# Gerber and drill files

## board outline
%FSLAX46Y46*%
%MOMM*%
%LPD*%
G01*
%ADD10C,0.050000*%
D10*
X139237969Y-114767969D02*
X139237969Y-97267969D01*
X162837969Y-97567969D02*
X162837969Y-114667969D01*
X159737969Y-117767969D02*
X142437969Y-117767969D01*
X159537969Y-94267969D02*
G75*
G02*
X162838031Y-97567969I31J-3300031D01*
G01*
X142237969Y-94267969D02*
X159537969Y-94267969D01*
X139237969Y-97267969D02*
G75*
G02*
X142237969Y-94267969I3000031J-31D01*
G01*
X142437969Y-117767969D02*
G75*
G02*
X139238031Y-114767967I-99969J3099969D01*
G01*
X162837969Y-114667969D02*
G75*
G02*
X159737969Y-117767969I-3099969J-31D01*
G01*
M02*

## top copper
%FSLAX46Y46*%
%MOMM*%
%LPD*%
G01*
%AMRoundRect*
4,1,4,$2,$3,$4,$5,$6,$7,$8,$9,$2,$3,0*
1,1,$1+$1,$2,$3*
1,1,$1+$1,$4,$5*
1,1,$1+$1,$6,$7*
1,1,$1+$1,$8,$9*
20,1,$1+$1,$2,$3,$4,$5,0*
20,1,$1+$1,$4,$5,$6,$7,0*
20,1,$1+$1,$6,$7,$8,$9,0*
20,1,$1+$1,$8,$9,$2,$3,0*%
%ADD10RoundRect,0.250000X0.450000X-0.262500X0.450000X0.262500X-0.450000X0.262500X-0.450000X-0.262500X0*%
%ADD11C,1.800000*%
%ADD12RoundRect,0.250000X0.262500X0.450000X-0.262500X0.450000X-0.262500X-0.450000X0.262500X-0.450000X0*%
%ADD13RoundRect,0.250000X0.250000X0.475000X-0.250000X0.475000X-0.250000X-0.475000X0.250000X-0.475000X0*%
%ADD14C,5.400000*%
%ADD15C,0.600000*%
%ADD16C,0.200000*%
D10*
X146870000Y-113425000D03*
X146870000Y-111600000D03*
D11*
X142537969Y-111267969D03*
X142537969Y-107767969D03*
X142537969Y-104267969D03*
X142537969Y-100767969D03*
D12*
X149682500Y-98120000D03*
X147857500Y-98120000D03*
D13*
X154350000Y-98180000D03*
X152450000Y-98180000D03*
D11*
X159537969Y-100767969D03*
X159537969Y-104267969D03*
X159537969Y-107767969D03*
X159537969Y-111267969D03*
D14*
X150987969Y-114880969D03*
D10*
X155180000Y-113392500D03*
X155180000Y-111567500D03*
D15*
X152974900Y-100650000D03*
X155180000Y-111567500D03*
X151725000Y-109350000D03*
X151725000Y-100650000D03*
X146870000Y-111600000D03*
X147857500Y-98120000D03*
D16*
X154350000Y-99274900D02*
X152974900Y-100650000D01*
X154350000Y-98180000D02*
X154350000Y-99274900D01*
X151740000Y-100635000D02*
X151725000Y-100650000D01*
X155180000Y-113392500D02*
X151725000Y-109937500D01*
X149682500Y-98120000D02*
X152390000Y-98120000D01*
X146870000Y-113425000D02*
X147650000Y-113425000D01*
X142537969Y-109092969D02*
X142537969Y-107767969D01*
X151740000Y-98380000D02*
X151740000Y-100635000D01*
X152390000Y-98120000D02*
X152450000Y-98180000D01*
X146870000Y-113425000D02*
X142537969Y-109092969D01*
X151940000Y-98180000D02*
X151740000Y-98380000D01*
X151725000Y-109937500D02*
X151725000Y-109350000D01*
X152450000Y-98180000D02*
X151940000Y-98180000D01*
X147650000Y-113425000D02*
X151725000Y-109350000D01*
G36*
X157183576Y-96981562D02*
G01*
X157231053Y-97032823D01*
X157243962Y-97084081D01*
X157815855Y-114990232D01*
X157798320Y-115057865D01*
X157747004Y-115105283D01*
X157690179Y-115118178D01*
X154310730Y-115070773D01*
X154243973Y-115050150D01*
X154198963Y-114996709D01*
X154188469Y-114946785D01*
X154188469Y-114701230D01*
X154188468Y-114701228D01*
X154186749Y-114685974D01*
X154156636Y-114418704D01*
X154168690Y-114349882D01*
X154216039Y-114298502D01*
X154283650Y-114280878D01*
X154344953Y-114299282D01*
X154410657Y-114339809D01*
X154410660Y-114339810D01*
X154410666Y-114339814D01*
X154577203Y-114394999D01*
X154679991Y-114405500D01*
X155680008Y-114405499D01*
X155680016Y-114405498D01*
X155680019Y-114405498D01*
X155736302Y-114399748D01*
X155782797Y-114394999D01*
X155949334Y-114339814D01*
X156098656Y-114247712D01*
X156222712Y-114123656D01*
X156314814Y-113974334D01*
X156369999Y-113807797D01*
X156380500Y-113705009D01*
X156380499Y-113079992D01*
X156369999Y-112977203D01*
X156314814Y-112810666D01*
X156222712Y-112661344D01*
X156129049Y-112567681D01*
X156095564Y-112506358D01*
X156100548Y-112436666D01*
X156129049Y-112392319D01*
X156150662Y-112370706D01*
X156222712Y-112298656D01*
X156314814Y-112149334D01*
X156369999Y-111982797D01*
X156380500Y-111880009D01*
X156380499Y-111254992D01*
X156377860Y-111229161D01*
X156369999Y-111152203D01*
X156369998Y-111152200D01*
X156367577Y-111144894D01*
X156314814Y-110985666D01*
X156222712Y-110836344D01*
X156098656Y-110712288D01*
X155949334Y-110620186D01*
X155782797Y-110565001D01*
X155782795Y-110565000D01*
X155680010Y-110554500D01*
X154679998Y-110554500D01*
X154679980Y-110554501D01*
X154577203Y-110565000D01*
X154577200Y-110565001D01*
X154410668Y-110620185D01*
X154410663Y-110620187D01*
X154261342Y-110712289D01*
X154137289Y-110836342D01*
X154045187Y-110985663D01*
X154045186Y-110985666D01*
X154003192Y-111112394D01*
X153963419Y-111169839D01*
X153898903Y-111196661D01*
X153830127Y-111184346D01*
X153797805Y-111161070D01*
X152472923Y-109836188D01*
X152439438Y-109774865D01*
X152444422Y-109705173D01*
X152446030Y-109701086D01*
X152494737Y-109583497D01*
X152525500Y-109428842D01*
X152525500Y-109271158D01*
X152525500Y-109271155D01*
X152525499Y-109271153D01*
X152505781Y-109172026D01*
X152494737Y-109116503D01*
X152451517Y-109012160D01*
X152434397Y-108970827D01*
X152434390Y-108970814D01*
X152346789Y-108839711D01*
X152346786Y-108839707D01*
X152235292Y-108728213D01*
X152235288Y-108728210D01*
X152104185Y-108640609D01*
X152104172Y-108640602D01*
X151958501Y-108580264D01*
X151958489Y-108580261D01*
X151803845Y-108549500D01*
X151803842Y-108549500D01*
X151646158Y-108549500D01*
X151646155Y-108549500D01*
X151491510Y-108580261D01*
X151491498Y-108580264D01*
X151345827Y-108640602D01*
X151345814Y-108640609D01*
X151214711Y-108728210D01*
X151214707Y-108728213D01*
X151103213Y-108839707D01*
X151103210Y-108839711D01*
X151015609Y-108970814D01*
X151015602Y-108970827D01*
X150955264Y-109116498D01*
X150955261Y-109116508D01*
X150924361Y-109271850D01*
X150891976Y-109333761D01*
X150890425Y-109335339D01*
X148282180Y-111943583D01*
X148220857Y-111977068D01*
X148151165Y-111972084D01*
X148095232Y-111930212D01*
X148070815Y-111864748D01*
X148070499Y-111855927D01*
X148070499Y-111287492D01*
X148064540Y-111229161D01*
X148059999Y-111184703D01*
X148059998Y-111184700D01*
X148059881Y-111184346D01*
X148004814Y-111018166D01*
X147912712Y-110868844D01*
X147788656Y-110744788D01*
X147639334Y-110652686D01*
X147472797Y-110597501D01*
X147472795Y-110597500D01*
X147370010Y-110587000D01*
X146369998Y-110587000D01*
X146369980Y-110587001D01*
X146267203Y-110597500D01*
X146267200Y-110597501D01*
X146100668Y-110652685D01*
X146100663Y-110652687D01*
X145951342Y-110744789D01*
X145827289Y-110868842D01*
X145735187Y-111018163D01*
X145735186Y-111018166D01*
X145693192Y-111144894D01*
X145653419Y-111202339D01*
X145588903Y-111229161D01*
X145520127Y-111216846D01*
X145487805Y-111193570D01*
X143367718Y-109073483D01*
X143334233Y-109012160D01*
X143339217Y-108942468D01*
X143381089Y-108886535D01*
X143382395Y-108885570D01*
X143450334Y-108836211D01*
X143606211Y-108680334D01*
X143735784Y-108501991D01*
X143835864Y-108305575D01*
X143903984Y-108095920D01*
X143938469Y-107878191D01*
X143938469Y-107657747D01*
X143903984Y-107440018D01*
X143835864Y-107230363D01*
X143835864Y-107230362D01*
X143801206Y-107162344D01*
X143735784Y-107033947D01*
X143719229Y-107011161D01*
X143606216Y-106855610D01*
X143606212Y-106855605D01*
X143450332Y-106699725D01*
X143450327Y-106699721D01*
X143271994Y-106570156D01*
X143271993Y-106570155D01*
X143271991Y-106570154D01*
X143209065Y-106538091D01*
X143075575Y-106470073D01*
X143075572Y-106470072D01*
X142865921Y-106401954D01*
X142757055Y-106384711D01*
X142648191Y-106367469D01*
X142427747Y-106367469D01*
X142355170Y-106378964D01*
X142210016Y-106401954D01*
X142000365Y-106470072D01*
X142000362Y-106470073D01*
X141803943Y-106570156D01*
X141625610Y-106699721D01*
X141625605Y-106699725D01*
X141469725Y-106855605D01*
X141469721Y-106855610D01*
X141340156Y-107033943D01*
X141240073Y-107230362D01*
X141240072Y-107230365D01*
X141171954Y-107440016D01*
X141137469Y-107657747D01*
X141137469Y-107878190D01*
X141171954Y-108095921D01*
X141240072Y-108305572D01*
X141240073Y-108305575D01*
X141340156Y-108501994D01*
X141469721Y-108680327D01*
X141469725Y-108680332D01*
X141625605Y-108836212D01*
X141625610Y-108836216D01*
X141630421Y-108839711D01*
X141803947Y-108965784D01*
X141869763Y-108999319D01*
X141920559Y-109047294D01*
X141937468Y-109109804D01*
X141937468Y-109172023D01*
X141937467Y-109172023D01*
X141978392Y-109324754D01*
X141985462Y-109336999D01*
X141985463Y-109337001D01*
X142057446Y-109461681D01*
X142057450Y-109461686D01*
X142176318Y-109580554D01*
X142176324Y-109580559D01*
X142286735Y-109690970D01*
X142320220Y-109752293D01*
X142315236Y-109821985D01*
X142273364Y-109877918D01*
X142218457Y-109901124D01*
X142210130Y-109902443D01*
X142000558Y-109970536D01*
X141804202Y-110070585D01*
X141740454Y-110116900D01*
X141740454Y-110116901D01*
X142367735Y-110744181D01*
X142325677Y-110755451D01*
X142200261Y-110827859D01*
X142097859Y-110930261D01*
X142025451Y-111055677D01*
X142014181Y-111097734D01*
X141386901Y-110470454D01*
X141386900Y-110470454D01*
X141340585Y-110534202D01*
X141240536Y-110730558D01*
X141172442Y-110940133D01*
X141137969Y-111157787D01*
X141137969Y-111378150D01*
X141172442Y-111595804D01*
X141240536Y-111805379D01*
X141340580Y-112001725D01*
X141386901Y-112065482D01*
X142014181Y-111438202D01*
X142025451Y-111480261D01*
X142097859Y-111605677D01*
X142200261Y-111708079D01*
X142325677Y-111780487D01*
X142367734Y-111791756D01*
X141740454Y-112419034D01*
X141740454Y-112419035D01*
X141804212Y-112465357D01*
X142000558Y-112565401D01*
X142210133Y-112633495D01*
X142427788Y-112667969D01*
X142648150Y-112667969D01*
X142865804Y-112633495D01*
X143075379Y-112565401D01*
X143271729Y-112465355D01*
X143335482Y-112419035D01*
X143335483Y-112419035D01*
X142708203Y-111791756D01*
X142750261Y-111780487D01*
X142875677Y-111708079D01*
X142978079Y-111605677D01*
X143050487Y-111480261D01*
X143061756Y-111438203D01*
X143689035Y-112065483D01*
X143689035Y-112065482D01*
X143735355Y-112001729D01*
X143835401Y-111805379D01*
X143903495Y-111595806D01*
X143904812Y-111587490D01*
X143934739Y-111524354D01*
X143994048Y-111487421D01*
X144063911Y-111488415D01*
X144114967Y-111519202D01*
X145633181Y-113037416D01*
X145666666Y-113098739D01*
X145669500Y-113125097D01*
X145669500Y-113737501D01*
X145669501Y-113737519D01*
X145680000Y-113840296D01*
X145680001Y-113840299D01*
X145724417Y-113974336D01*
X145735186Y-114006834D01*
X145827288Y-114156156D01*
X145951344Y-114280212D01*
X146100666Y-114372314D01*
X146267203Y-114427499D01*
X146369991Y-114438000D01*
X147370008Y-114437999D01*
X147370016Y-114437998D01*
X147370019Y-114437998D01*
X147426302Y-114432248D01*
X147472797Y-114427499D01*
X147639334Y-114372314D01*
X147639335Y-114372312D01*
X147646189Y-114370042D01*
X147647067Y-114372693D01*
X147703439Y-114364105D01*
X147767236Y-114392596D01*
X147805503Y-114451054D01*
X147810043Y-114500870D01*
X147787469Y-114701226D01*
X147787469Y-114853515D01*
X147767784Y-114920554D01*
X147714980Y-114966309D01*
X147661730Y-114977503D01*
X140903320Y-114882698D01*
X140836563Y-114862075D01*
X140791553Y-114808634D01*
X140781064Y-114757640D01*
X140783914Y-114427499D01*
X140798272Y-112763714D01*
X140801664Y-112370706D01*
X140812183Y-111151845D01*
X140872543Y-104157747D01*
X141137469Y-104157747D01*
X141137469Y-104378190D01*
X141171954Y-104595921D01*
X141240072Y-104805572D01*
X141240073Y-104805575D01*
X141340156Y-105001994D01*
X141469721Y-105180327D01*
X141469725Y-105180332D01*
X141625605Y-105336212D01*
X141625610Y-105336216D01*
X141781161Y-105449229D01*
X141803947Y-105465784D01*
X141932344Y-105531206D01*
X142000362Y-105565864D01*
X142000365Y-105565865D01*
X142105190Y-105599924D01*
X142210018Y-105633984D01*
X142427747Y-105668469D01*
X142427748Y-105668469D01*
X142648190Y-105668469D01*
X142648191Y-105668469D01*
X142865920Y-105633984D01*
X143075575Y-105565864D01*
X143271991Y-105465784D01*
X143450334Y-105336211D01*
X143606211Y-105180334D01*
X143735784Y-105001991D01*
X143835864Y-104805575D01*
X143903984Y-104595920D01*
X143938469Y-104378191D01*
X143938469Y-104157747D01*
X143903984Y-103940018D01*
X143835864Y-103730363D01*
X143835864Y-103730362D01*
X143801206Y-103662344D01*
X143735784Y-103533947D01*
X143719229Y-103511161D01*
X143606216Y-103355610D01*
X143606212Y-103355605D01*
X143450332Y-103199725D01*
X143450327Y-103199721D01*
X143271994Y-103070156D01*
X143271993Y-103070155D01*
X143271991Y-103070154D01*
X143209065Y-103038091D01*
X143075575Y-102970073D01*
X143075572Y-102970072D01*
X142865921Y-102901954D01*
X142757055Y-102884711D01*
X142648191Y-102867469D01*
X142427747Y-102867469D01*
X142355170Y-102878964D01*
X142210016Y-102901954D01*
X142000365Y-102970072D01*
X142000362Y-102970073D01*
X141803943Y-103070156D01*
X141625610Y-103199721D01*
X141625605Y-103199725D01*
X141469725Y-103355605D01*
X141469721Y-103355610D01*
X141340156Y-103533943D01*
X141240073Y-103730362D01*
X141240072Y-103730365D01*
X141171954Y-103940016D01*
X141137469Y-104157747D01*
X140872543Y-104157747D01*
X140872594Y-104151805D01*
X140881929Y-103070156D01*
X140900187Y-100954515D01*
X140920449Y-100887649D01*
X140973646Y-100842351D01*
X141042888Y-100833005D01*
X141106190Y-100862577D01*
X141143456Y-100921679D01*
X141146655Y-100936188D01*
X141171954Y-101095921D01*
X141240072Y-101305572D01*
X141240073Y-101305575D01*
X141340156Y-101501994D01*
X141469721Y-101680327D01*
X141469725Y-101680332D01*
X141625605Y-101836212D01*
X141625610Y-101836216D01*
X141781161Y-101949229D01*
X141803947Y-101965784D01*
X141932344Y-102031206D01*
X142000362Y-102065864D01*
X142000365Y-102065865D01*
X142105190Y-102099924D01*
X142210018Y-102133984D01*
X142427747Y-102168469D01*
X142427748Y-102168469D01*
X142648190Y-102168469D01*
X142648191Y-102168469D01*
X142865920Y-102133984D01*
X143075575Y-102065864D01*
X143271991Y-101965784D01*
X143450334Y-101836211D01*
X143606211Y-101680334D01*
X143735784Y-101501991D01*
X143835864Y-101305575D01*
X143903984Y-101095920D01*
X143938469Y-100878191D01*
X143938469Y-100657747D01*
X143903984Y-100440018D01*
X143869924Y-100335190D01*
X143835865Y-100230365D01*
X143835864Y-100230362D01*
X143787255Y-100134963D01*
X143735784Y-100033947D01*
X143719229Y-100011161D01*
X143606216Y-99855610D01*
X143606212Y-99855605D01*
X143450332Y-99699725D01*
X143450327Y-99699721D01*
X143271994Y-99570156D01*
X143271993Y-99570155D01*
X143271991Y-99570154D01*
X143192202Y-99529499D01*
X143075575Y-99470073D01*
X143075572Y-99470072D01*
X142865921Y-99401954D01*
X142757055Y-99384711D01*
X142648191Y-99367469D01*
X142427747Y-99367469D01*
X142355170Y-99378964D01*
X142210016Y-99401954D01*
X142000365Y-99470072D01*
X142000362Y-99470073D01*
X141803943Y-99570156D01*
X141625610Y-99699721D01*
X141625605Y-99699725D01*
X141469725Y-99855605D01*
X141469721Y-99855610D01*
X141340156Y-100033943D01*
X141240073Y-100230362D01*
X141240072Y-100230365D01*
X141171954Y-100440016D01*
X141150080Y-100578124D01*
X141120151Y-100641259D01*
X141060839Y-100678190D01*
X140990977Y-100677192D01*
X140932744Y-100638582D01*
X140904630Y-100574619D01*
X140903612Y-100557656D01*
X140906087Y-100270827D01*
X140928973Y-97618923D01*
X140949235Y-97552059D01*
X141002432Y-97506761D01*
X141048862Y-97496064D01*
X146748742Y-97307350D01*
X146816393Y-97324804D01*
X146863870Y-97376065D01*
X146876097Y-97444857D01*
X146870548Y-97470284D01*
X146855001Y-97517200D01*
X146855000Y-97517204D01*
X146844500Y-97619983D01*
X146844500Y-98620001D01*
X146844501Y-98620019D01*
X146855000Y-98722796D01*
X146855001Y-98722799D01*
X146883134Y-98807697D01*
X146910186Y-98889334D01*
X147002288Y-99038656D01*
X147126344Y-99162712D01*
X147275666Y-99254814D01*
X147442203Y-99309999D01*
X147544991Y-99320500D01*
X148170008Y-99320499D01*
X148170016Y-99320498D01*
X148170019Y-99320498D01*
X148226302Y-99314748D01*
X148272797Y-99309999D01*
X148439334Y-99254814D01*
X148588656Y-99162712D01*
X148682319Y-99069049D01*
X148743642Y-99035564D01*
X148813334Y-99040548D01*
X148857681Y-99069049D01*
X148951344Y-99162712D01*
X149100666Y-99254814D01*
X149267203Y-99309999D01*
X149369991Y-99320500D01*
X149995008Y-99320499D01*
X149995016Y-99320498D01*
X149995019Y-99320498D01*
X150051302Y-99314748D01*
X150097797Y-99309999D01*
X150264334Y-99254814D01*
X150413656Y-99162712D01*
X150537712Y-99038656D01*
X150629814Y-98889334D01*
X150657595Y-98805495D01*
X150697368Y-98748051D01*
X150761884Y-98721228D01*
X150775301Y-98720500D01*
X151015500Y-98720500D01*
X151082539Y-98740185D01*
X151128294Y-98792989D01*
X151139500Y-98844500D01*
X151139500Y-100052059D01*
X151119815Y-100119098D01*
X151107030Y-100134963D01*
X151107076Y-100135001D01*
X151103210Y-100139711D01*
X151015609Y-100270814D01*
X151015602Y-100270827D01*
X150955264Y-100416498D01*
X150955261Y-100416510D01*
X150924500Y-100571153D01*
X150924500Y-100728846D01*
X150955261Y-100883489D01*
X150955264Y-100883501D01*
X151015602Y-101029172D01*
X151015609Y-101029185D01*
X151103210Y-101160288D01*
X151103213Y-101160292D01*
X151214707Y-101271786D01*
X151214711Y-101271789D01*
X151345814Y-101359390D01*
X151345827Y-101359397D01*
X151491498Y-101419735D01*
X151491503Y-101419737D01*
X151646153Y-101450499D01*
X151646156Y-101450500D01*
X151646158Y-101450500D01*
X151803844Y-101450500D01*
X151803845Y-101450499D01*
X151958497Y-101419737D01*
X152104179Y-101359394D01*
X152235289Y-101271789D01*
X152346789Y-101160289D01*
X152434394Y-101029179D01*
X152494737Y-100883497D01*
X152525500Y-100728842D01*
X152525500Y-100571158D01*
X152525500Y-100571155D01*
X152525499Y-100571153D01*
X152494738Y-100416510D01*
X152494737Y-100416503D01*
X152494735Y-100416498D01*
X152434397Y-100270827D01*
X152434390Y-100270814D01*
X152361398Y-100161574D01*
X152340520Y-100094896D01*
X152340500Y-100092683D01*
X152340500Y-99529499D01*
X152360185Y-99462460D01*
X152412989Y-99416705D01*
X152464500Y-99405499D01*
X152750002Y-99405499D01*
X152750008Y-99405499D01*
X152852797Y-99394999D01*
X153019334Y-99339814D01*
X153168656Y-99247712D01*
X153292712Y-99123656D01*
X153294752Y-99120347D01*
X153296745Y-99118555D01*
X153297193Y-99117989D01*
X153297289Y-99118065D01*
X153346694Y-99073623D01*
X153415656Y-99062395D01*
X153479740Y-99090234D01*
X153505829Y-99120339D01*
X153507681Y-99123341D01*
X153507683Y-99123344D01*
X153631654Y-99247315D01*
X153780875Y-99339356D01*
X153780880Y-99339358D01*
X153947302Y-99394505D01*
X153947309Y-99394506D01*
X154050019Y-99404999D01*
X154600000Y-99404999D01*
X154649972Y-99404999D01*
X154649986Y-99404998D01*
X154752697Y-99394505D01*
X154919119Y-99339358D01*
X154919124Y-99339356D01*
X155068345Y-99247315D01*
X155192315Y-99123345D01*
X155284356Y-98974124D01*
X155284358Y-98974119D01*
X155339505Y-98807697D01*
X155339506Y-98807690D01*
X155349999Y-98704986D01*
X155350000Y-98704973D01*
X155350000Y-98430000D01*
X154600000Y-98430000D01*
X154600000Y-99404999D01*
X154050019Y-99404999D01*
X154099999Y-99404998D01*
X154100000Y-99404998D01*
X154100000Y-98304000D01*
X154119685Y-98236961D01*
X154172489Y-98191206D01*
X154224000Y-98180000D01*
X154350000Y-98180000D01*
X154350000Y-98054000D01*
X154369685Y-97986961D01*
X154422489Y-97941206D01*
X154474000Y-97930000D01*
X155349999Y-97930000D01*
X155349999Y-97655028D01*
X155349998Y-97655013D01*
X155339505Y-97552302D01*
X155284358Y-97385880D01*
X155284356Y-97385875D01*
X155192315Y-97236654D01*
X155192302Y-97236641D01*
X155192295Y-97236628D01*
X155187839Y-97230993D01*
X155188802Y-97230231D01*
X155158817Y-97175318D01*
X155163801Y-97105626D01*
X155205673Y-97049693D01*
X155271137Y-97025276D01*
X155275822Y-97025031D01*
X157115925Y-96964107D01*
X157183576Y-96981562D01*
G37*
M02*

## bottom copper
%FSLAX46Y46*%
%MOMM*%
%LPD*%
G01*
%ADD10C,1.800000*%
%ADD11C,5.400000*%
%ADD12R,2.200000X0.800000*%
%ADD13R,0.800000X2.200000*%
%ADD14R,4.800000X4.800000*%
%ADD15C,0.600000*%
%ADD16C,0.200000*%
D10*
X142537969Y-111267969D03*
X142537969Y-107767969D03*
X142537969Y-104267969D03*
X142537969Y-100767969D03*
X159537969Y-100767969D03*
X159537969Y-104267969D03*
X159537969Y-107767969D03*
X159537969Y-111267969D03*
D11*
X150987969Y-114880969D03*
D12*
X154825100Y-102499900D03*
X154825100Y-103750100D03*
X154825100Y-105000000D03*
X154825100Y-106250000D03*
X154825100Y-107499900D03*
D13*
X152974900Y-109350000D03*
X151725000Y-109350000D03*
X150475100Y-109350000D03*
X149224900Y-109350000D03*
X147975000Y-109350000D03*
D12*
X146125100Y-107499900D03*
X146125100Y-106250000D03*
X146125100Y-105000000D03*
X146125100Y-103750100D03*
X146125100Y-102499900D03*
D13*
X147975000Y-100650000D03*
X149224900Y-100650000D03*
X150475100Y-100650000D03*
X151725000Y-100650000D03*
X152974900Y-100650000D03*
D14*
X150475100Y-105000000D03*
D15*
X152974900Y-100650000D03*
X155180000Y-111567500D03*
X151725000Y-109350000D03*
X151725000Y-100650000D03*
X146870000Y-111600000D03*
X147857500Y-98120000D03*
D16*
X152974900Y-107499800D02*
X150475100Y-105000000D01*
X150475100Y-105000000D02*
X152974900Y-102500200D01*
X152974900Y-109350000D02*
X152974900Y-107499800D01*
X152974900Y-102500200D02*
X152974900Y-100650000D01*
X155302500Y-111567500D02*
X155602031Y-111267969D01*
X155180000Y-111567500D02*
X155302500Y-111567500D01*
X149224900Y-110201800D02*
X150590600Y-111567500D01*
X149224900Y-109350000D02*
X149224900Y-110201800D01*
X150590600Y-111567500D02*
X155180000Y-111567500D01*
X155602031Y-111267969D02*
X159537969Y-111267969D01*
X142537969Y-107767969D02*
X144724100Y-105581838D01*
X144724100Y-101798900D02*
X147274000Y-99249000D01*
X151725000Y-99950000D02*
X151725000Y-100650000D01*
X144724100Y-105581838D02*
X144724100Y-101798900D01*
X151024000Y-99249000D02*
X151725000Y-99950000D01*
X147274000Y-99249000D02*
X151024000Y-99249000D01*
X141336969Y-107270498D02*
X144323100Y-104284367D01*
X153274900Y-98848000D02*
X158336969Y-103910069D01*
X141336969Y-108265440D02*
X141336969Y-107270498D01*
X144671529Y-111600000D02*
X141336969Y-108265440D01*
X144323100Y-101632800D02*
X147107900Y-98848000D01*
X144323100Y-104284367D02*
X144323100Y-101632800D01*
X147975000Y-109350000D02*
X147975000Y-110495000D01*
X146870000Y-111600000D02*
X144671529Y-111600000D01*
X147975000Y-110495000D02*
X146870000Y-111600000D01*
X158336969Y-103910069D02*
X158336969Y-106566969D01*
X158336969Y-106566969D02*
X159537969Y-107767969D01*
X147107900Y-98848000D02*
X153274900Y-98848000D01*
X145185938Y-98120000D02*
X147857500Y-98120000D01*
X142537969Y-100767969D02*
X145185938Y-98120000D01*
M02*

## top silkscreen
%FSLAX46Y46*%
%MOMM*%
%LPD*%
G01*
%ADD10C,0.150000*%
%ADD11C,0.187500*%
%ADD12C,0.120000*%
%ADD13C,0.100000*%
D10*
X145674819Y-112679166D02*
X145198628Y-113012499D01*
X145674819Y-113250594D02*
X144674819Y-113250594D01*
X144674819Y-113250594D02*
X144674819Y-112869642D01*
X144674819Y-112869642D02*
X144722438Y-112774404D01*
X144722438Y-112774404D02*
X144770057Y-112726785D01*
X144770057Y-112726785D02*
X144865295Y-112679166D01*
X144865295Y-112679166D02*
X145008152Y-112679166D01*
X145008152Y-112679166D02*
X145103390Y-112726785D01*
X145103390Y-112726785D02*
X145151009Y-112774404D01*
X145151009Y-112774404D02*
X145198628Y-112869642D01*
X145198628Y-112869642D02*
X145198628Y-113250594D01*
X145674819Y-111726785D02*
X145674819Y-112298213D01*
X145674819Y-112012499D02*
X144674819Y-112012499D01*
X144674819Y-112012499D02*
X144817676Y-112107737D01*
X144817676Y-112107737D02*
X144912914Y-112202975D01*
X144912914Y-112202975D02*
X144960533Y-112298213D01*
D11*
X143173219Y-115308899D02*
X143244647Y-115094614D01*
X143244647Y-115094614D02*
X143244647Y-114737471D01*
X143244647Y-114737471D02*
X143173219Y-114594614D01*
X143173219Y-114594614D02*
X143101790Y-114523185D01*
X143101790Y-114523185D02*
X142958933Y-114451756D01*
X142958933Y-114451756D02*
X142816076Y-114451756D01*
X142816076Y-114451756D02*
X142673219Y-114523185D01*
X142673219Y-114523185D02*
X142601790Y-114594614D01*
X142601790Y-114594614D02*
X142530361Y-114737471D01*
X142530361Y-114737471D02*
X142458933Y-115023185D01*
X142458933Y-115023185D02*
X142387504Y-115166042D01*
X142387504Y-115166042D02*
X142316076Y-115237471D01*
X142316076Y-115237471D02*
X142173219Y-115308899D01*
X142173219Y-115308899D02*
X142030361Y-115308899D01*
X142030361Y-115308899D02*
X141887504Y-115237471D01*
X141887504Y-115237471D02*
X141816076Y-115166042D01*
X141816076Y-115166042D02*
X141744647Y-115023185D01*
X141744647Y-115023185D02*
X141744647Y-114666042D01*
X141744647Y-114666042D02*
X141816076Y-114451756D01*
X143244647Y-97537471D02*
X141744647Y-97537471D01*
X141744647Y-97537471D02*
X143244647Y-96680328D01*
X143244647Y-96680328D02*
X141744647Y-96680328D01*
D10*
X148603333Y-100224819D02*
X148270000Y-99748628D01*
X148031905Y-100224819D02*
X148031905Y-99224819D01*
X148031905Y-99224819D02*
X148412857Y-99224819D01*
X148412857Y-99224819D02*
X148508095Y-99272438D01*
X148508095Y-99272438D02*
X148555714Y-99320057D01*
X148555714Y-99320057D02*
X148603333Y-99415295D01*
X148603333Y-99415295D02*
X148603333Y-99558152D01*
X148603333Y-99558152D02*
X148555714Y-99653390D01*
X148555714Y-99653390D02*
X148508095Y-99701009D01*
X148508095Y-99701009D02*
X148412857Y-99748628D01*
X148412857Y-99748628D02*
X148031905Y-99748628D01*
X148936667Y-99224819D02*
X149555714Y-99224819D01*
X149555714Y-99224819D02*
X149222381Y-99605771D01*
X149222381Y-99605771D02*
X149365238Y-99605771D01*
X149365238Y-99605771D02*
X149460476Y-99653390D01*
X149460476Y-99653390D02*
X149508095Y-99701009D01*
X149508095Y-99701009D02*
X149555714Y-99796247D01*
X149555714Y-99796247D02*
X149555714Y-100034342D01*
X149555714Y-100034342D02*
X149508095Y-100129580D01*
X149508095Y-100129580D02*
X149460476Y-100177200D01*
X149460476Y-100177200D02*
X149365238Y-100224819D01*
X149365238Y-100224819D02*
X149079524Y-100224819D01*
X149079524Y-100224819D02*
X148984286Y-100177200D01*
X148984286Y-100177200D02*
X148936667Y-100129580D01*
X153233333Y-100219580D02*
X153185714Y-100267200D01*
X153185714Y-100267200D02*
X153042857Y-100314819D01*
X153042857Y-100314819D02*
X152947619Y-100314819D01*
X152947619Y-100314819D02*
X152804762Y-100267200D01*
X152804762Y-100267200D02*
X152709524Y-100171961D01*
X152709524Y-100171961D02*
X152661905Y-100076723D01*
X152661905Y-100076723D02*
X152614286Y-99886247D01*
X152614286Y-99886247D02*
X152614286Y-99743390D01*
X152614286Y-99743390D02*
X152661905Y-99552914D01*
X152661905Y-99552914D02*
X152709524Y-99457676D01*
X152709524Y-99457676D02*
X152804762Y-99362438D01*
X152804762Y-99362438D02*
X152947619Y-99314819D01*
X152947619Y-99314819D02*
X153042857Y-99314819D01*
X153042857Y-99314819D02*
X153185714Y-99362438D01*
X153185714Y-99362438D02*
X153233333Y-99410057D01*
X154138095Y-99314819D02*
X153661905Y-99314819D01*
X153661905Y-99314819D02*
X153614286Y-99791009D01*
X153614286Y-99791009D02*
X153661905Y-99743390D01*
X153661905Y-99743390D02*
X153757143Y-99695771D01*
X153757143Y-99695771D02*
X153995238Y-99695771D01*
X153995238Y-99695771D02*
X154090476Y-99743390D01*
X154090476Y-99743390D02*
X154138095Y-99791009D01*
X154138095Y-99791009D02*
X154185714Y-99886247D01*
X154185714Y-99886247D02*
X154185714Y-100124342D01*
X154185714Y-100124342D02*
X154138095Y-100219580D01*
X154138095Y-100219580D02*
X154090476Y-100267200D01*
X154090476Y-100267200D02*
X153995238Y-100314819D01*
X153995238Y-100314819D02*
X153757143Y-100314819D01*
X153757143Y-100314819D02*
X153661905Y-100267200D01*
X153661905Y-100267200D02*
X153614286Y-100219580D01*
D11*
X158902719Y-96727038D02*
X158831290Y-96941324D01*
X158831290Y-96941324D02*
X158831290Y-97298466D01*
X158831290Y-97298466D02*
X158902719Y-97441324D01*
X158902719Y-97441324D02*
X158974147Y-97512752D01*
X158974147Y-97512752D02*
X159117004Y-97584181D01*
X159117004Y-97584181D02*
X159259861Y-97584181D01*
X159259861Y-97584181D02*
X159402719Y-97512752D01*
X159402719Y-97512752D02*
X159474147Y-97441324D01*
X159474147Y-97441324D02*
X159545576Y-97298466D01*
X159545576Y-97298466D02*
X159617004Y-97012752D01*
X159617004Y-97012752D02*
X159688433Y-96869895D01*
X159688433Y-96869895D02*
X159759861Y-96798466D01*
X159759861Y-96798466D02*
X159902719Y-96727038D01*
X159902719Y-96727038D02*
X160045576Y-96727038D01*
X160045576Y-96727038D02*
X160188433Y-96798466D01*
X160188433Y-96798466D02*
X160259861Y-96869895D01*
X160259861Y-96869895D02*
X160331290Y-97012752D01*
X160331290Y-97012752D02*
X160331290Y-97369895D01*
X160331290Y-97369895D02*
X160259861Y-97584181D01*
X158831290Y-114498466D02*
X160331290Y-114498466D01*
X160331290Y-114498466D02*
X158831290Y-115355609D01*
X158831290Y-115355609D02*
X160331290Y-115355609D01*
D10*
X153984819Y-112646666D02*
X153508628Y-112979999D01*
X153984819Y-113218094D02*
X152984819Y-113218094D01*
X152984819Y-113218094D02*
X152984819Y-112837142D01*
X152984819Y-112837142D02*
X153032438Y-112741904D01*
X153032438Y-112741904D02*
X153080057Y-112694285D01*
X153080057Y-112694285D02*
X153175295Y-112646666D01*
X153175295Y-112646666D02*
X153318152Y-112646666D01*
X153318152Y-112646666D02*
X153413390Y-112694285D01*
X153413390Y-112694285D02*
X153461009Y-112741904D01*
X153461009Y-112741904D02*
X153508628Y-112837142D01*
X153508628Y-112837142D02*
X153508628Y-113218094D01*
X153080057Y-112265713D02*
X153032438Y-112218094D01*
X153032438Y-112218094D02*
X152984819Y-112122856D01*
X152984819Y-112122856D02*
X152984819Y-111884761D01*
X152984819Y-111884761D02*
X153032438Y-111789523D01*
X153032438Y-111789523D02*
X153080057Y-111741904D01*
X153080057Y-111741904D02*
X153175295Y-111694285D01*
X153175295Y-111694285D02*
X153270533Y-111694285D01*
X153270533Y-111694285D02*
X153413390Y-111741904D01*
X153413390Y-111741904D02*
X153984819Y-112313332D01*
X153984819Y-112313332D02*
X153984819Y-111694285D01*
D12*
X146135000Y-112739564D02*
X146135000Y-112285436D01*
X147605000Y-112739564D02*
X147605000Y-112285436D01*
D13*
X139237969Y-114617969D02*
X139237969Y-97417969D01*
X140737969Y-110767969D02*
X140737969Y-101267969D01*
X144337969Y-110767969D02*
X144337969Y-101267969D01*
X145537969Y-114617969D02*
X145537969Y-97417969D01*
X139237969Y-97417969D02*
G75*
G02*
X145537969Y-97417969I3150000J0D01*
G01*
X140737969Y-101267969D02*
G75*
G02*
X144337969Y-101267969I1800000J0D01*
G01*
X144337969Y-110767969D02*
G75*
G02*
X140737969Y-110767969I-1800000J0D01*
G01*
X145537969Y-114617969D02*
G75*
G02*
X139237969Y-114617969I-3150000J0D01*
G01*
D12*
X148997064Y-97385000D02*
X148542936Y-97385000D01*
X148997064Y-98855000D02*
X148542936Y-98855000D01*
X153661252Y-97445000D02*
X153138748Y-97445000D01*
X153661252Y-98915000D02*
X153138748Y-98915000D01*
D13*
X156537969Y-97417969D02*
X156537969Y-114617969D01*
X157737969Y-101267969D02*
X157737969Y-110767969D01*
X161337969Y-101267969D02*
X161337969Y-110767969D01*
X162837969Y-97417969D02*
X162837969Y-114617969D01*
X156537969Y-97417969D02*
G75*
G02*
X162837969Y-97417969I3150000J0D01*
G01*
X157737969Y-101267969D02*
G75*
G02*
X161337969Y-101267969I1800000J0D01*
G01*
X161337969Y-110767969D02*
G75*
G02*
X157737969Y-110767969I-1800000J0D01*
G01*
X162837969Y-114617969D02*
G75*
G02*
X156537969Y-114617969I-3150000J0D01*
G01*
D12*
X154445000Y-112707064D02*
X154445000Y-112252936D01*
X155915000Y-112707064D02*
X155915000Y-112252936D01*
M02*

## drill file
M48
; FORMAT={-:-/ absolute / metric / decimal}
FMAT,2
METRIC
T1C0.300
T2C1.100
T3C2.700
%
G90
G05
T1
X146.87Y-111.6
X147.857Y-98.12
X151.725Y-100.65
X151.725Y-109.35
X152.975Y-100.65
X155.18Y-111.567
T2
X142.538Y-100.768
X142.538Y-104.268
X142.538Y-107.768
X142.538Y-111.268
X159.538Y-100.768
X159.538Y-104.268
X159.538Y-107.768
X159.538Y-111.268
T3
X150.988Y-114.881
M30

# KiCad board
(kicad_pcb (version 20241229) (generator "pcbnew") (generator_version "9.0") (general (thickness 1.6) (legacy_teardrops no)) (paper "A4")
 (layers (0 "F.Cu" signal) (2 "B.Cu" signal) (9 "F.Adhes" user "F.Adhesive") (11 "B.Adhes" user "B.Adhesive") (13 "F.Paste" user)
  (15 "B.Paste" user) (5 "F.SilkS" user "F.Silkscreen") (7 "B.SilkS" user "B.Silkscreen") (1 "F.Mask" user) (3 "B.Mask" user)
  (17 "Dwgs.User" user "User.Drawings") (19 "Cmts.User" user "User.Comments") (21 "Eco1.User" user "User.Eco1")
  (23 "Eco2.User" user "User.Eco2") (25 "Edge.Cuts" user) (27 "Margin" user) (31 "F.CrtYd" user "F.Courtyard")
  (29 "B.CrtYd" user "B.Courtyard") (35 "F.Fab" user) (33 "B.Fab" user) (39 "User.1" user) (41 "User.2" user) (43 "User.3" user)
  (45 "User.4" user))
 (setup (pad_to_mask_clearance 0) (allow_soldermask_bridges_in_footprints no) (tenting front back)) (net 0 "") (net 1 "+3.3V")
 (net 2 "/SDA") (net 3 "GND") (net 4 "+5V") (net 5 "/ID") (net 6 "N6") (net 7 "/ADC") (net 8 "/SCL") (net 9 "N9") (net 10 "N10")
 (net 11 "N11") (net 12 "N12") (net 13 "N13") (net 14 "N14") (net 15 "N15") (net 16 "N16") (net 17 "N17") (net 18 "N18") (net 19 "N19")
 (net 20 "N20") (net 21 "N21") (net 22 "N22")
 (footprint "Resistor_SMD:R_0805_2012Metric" (layer "F.Cu") (at 146.87 112.5125 90)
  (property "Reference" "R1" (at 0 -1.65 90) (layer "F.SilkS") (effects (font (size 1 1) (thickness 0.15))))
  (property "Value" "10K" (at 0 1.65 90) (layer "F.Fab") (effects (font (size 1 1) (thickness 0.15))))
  (fp_line (start -0.227064 -0.735) (end 0.227064 -0.735) (stroke (width 0.12) (type solid)) (layer "F.SilkS"))
  (fp_line (start -0.227064 0.735) (end 0.227064 0.735) (stroke (width 0.12) (type solid)) (layer "F.SilkS"))
  (pad "1" smd roundrect (at -0.9125 0 90) (size 1.025 1.4) (layers "F.Cu" "F.Mask" "F.Paste") (roundrect_rratio 0.243902) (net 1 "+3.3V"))
  (pad "2" smd roundrect (at 0.9125 0 90) (size 1.025 1.4) (layers "F.Cu" "F.Mask" "F.Paste") (roundrect_rratio 0.243902) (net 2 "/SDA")))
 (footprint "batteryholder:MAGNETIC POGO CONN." (layer "F.Cu") (at 142.537969 106.017969 90)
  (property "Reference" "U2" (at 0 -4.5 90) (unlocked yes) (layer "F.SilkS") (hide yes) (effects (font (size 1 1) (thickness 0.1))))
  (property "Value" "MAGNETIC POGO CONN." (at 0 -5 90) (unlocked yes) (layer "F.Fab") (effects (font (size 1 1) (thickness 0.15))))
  (fp_line (start -8.6 -3.3) (end 8.6 -3.3) (stroke (width 0.1) (type default)) (layer "F.SilkS"))
  (fp_line (start -4.75 -1.8) (end 4.75 -1.8) (stroke (width 0.1) (type default)) (layer "F.SilkS"))
  (fp_line (start -4.75 1.8) (end 4.75 1.8) (stroke (width 0.1) (type default)) (layer "F.SilkS"))
  (fp_line (start -8.6 3) (end 8.6 3) (stroke (width 0.1) (type default)) (layer "F.SilkS"))
  (fp_arc (start 8.6 -3.3) (mid 11.75 -0.15) (end 8.6 3) (stroke (width 0.1) (type default)) (layer "F.SilkS"))
  (fp_arc (start 4.75 -1.8) (mid 6.55 0) (end 4.75 1.8) (stroke (width 0.1) (type default)) (layer "F.SilkS"))
  (fp_arc (start -4.75 1.8) (mid -6.55 0) (end -4.75 -1.8) (stroke (width 0.1) (type default)) (layer "F.SilkS"))
  (fp_arc (start -8.6 3) (mid -11.75 -0.15) (end -8.6 -3.3) (stroke (width 0.1) (type default)) (layer "F.SilkS"))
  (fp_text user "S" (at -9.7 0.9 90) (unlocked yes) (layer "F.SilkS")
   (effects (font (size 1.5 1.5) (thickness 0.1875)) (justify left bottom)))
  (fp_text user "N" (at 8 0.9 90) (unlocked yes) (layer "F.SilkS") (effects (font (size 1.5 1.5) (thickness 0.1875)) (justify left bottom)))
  (pad "1" thru_hole circle (at -5.25 0 90) (size 1.8 1.8) (drill 1.1) (layers "*.Cu" "*.Mask") (remove_unused_layers no) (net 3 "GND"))
  (pad "2" thru_hole circle (at -1.75 0 90) (size 1.8 1.8) (drill 1.1) (layers "*.Cu" "*.Mask") (remove_unused_layers no) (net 1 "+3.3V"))
  (pad "3" thru_hole circle (at 1.75 0 90) (size 1.8 1.8) (drill 1.1) (layers "*.Cu" "*.Mask") (remove_unused_layers no) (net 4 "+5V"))
  (pad "4" thru_hole circle (at 5.25 0 90) (size 1.8 1.8) (drill 1.1) (layers "*.Cu" "*.Mask") (remove_unused_layers no) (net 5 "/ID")))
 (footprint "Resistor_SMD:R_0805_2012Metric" (layer "F.Cu") (at 148.77 98.12 180)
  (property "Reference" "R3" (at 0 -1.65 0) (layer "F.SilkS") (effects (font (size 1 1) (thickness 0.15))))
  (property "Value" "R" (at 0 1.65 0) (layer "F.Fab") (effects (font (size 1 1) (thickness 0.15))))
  (fp_line (start -0.227064 0.735) (end 0.227064 0.735) (stroke (width 0.12) (type solid)) (layer "F.SilkS"))
  (fp_line (start -0.227064 -0.735) (end 0.227064 -0.735) (stroke (width 0.12) (type solid)) (layer "F.SilkS"))
  (pad "1" smd roundrect (at -0.9125 0 180) (size 1.025 1.4) (layers "F.Cu" "F.Mask" "F.Paste") (roundrect_rratio 0.243902) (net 1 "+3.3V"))
  (pad "2" smd roundrect (at 0.9125 0 180) (size 1.025 1.4) (layers "F.Cu" "F.Mask" "F.Paste") (roundrect_rratio 0.243902) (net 5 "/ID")))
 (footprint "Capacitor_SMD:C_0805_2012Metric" (layer "F.Cu") (at 153.4 98.18 180)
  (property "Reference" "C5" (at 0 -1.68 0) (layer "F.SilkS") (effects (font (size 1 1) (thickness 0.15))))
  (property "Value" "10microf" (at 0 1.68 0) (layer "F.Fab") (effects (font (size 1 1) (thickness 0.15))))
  (fp_line (start -0.261252 0.735) (end 0.261252 0.735) (stroke (width 0.12) (type solid)) (layer "F.SilkS"))
  (fp_line (start -0.261252 -0.735) (end 0.261252 -0.735) (stroke (width 0.12) (type solid)) (layer "F.SilkS"))
  (pad "1" smd roundrect (at -0.95 0 180) (size 1 1.45) (layers "F.Cu" "F.Mask" "F.Paste") (roundrect_rratio 0.25) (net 3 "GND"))
  (pad "2" smd roundrect (at 0.95 0 180) (size 1 1.45) (layers "F.Cu" "F.Mask" "F.Paste") (roundrect_rratio 0.25) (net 1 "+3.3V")))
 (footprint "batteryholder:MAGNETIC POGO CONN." (layer "F.Cu") (at 159.537969 106.017969 -90)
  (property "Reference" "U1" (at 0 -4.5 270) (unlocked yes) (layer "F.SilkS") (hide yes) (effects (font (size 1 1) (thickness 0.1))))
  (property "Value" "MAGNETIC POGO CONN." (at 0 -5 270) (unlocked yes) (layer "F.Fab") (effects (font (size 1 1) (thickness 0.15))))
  (fp_line (start -8.6 3) (end 8.6 3) (stroke (width 0.1) (type default)) (layer "F.SilkS"))
  (fp_line (start -4.75 1.8) (end 4.75 1.8) (stroke (width 0.1) (type default)) (layer "F.SilkS"))
  (fp_line (start -4.75 -1.8) (end 4.75 -1.8) (stroke (width 0.1) (type default)) (layer "F.SilkS"))
  (fp_line (start -8.6 -3.3) (end 8.6 -3.3) (stroke (width 0.1) (type default)) (layer "F.SilkS"))
  (fp_arc (start -8.6 3) (mid -11.75 -0.15) (end -8.6 -3.3) (stroke (width 0.1) (type default)) (layer "F.SilkS"))
  (fp_arc (start -4.75 1.8) (mid -6.55 0) (end -4.75 -1.8) (stroke (width 0.1) (type default)) (layer "F.SilkS"))
  (fp_arc (start 4.75 -1.8) (mid 6.55 0) (end 4.75 1.8) (stroke (width 0.1) (type default)) (layer "F.SilkS"))
  (fp_arc (start 8.6 -3.3) (mid 11.75 -0.15) (end 8.6 3) (stroke (width 0.1) (type default)) (layer "F.SilkS"))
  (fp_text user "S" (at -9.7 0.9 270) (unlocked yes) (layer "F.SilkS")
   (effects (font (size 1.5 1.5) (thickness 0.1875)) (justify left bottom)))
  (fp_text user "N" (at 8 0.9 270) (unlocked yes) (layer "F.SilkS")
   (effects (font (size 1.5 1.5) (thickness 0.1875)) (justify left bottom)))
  (pad "1" thru_hole circle (at -5.25 0 270) (size 1.8 1.8) (drill 1.1) (layers "*.Cu" "*.Mask") (remove_unused_layers no) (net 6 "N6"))
  (pad "2" thru_hole circle (at -1.75 0 270) (size 1.8 1.8) (drill 1.1) (layers "*.Cu" "*.Mask") (remove_unused_layers no) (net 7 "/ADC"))
  (pad "3" thru_hole circle (at 1.75 0 270) (size 1.8 1.8) (drill 1.1) (layers "*.Cu" "*.Mask") (remove_unused_layers no) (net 2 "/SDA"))
  (pad "4" thru_hole circle (at 5.25 0 270) (size 1.8 1.8) (drill 1.1) (layers "*.Cu" "*.Mask") (remove_unused_layers no) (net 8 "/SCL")))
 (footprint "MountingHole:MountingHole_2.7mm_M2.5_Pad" (layer "F.Cu") (at 150.987969 114.880969)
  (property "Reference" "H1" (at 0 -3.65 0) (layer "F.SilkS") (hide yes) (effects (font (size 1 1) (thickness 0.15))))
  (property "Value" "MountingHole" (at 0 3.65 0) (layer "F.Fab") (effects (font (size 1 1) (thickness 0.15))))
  (pad "1" thru_hole circle (at 0 0) (size 5.4 5.4) (drill 2.7) (layers "*.Cu" "*.Mask") (remove_unused_layers no) (zone_connect 2)))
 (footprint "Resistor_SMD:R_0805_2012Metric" (layer "F.Cu") (at 155.18 112.48 90)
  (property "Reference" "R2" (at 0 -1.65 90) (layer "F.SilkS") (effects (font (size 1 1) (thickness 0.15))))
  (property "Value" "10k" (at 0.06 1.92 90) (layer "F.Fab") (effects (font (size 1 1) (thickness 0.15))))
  (fp_line (start -0.227064 -0.735) (end 0.227064 -0.735) (stroke (width 0.12) (type solid)) (layer "F.SilkS"))
  (fp_line (start -0.227064 0.735) (end 0.227064 0.735) (stroke (width 0.12) (type solid)) (layer "F.SilkS"))
  (pad "1" smd roundrect (at -0.9125 0 90) (size 1.025 1.4) (layers "F.Cu" "F.Mask" "F.Paste") (roundrect_rratio 0.243902) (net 1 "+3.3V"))
  (pad "2" smd roundrect (at 0.9125 0 90) (size 1.025 1.4) (layers "F.Cu" "F.Mask" "F.Paste") (roundrect_rratio 0.243902) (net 8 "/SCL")))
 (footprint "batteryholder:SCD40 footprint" (layer "B.Cu") (at 150.475 105 180)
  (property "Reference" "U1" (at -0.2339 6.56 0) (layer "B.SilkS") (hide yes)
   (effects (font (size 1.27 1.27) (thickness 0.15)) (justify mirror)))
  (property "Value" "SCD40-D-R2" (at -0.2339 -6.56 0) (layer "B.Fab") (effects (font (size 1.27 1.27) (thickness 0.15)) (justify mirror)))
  (pad "1" smd rect (at -4.3501 2.5001 180) (size 2.2 0.8) (layers "B.Cu" "B.Mask" "B.Paste") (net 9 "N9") (solder_mask_margin 0.05)
   (solder_paste_margin 0) (thermal_bridge_angle 0))
  (pad "2" smd rect (at -4.3501 1.2499 180) (size 2.2 0.8) (layers "B.Cu" "B.Mask" "B.Paste") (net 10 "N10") (solder_mask_margin 0.05)
   (solder_paste_margin 0) (thermal_bridge_angle 0))
  (pad "3" smd rect (at -4.3501 0 180) (size 2.2 0.8) (layers "B.Cu" "B.Mask" "B.Paste") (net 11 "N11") (solder_mask_margin 0.05)
   (solder_paste_margin 0) (thermal_bridge_angle 0))
  (pad "4" smd rect (at -4.3501 -1.25 180) (size 2.2 0.8) (layers "B.Cu" "B.Mask" "B.Paste") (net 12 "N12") (solder_mask_margin 0.05)
   (solder_paste_margin 0) (thermal_bridge_angle 0))
  (pad "5" smd rect (at -4.3501 -2.4999 180) (size 2.2 0.8) (layers "B.Cu" "B.Mask" "B.Paste") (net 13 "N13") (solder_mask_margin 0.05)
   (solder_paste_margin 0) (thermal_bridge_angle 0))
  (pad "6" smd rect (at -2.4999 -4.35 90) (size 2.2 0.8) (layers "B.Cu" "B.Mask" "B.Paste") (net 3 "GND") (solder_mask_margin 0.05)
   (solder_paste_margin 0) (thermal_bridge_angle 0))
  (pad "7" smd rect (at -1.25 -4.35 90) (size 2.2 0.8) (layers "B.Cu" "B.Mask" "B.Paste") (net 1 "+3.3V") (solder_mask_margin 0.05)
   (solder_paste_margin 0) (thermal_bridge_angle 0))
  (pad "8" smd rect (at -0.0001 -4.35 90) (size 2.2 0.8) (layers "B.Cu" "B.Mask" "B.Paste") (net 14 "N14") (solder_mask_margin 0.05)
   (solder_paste_margin 0) (thermal_bridge_angle 0))
  (pad "9" smd rect (at 1.2501 -4.35 90) (size 2.2 0.8) (layers "B.Cu" "B.Mask" "B.Paste") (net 8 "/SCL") (solder_mask_margin 0.05)
   (solder_paste_margin 0) (thermal_bridge_angle 0))
  (pad "10" smd rect (at 2.5 -4.35 90) (size 2.2 0.8) (layers "B.Cu" "B.Mask" "B.Paste") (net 2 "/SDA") (solder_mask_margin 0.05)
   (solder_paste_margin 0) (thermal_bridge_angle 0))
  (pad "11" smd rect (at 4.3499 -2.4999) (size 2.2 0.8) (layers "B.Cu" "B.Mask" "B.Paste") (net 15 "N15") (solder_mask_margin 0.05)
   (solder_paste_margin 0) (thermal_bridge_angle 0))
  (pad "12" smd rect (at 4.3499 -1.25) (size 2.2 0.8) (layers "B.Cu" "B.Mask" "B.Paste") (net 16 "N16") (solder_mask_margin 0.05)
   (solder_paste_margin 0) (thermal_bridge_angle 0))
  (pad "13" smd rect (at 4.3499 0) (size 2.2 0.8) (layers "B.Cu" "B.Mask" "B.Paste") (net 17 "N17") (solder_mask_margin 0.05)
   (solder_paste_margin 0) (thermal_bridge_angle 0))
  (pad "14" smd rect (at 4.3499 1.2499) (size 2.2 0.8) (layers "B.Cu" "B.Mask" "B.Paste") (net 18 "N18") (solder_mask_margin 0.05)
   (solder_paste_margin 0) (thermal_bridge_angle 0))
  (pad "15" smd rect (at 4.3499 2.5001) (size 2.2 0.8) (layers "B.Cu" "B.Mask" "B.Paste") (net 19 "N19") (solder_mask_margin 0.05)
   (solder_paste_margin 0) (thermal_bridge_angle 0))
  (pad "16" smd rect (at 2.5 4.35 270) (size 2.2 0.8) (layers "B.Cu" "B.Mask" "B.Paste") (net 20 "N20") (solder_mask_margin 0.05)
   (solder_paste_margin 0) (thermal_bridge_angle 0))
  (pad "17" smd rect (at 1.2501 4.35 270) (size 2.2 0.8) (layers "B.Cu" "B.Mask" "B.Paste") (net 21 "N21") (solder_mask_margin 0.05)
   (solder_paste_margin 0) (thermal_bridge_angle 0))
  (pad "18" smd rect (at -0.0001 4.35 270) (size 2.2 0.8) (layers "B.Cu" "B.Mask" "B.Paste") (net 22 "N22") (solder_mask_margin 0.05)
   (solder_paste_margin 0) (thermal_bridge_angle 0))
  (pad "19" smd rect (at -1.25 4.35 270) (size 2.2 0.8) (layers "B.Cu" "B.Mask" "B.Paste") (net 1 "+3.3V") (solder_mask_margin 0.05)
   (solder_paste_margin 0) (thermal_bridge_angle 0))
  (pad "20" smd rect (at -2.4999 4.35 270) (size 2.2 0.8) (layers "B.Cu" "B.Mask" "B.Paste") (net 3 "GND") (solder_mask_margin 0.05)
   (solder_paste_margin 0) (thermal_bridge_angle 0))
  (pad "21" smd rect (at -0.0001 0 90) (size 4.8 4.8) (layers "B.Cu" "B.Mask" "B.Paste") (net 3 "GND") (solder_mask_margin 0.05)
   (solder_paste_margin 0) (thermal_bridge_angle 0))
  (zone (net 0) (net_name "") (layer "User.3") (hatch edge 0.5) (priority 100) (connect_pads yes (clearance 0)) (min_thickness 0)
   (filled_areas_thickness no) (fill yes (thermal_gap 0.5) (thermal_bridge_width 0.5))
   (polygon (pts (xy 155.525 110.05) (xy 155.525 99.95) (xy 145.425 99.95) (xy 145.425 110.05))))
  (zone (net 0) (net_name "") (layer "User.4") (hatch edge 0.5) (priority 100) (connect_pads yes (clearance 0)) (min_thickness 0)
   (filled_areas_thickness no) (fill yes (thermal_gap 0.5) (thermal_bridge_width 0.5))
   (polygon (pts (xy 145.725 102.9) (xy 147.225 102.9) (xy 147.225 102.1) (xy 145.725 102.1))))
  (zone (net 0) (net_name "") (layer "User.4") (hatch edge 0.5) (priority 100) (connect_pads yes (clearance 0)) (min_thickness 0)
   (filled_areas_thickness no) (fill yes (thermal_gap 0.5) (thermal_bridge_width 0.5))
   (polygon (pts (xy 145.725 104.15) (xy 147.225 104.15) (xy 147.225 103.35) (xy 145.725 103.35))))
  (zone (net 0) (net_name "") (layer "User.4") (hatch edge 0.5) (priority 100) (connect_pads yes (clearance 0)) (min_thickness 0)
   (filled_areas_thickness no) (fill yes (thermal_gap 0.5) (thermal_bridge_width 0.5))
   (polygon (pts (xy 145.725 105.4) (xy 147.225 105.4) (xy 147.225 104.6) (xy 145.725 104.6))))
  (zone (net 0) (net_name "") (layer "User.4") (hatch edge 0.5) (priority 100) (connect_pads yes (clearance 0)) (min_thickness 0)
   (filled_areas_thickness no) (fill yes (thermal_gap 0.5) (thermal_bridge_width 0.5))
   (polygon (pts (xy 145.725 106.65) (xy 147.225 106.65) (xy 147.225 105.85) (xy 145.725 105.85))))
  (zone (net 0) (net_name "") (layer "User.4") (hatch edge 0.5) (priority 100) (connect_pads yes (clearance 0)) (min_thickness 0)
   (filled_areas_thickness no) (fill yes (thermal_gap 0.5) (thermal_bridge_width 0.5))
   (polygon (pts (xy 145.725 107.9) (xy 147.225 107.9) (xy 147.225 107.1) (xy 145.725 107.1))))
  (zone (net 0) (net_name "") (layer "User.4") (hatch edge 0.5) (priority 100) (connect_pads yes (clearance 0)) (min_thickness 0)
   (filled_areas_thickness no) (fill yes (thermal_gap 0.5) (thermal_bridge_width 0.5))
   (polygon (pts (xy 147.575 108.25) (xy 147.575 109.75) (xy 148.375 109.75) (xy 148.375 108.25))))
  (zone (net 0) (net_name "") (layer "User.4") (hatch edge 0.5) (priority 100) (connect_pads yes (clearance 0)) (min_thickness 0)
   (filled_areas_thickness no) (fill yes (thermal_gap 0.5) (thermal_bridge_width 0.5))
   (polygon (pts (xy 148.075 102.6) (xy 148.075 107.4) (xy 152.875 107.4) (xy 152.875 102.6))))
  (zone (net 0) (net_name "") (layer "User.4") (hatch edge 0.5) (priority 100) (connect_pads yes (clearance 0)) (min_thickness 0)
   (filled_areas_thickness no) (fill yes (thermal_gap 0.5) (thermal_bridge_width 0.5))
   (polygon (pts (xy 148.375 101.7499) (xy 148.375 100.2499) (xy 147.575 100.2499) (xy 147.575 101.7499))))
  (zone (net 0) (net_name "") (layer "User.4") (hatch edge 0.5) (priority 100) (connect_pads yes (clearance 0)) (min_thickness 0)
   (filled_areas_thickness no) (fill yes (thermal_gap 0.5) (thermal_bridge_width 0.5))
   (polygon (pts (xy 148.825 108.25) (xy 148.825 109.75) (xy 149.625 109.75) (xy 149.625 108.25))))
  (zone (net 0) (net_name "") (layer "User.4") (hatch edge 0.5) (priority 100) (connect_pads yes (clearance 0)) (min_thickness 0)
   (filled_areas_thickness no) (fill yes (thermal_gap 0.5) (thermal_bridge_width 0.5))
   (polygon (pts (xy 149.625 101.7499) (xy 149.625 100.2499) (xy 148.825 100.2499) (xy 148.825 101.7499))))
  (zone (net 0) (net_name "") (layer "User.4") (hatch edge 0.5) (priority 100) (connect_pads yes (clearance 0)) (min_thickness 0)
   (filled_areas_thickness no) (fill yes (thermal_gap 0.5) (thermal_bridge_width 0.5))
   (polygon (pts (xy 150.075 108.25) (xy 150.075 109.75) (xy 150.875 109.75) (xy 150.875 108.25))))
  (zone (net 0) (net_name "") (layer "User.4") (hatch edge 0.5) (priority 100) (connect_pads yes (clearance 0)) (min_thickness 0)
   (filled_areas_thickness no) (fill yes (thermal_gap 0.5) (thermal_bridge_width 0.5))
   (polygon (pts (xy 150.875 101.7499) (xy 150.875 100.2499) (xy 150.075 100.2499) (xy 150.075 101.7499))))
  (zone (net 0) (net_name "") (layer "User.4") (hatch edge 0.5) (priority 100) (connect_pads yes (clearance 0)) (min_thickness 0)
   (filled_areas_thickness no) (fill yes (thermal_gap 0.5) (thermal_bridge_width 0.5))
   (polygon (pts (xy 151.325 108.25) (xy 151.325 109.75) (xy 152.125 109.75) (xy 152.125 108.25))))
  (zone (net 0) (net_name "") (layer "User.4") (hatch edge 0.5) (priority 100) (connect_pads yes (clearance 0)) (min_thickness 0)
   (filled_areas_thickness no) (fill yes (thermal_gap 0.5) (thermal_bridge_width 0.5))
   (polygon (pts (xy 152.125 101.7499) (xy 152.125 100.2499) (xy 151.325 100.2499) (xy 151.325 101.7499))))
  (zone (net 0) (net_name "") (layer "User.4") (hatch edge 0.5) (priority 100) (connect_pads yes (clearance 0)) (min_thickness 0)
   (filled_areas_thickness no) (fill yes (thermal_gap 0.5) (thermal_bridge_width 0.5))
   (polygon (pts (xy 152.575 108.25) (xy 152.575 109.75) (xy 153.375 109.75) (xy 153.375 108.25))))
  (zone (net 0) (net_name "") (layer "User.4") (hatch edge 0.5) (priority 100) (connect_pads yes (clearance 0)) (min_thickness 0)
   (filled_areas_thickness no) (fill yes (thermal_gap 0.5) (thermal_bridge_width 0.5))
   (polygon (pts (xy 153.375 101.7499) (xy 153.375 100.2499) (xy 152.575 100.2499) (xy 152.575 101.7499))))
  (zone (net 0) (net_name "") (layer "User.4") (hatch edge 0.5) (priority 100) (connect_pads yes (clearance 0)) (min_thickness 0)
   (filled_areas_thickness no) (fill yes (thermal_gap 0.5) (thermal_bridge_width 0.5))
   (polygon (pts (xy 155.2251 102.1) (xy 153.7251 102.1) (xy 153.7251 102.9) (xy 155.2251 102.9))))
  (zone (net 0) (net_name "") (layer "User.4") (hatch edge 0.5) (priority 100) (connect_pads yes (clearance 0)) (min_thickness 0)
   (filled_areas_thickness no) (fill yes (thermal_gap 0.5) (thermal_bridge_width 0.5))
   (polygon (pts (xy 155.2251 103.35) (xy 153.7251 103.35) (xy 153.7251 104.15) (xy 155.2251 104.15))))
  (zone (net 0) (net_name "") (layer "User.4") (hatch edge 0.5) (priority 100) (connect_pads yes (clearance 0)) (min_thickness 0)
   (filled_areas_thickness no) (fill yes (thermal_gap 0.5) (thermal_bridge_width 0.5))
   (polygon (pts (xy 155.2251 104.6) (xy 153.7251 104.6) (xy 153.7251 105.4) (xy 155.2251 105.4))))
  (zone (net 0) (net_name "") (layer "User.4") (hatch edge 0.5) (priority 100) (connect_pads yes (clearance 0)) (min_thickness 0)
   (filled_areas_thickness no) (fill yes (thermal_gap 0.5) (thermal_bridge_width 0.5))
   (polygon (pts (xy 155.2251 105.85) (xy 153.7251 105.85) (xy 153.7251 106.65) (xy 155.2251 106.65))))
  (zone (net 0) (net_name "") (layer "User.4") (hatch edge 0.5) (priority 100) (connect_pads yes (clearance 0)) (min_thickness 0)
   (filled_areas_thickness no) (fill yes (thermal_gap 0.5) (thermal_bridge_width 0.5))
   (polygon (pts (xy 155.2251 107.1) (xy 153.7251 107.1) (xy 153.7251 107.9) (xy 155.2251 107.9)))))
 (gr_line (start 139.237969 114.767969) (end 139.237969 97.267969) (stroke (width 0.05) (type default)) (layer "Edge.Cuts"))
 (gr_line (start 162.837969 97.567969) (end 162.837969 114.667969) (stroke (width 0.05) (type default)) (layer "Edge.Cuts"))
 (gr_line (start 159.737969 117.767969) (end 142.437969 117.767969) (stroke (width 0.05) (type solid)) (layer "Edge.Cuts"))
 (gr_arc (start 159.537969 94.267969) (mid 161.871421 95.234517) (end 162.837969 97.567969) (stroke (width 0.05) (type default))
  (layer "Edge.Cuts"))
 (gr_line (start 142.237969 94.267969) (end 159.537969 94.267969) (stroke (width 0.05) (type default)) (layer "Edge.Cuts"))
 (gr_arc (start 139.237969 97.267969) (mid 140.116649 95.146649) (end 142.237969 94.267969) (stroke (width 0.05) (type default))
  (layer "Edge.Cuts"))
 (gr_arc (start 142.437969 117.767969) (mid 140.216649 116.930711) (end 139.237969 114.767969) (stroke (width 0.05) (type default))
  (layer "Edge.Cuts"))
 (gr_arc (start 162.837969 114.667969) (mid 161.93 116.86) (end 159.737969 117.767969) (stroke (width 0.05) (type default))
  (layer "Edge.Cuts"))
 (segment (start 154.35 99.2749) (end 152.9749 100.65) (width 0.2) (layer "F.Cu") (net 3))
 (segment (start 154.35 98.18) (end 154.35 99.2749) (width 0.2) (layer "F.Cu") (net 3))
 (via blind (at 152.9749 100.65) (size 0.6) (drill 0.3) (layers "F.Cu" "B.Cu") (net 3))
 (segment (start 152.9749 107.4998) (end 150.4751 105) (width 0.2) (layer "B.Cu") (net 3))
 (segment (start 150.4751 105) (end 152.9749 102.5002) (width 0.2) (layer "B.Cu") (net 3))
 (segment (start 152.9749 109.35) (end 152.9749 107.4998) (width 0.2) (layer "B.Cu") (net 3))
 (segment (start 152.9749 102.5002) (end 152.9749 100.65) (width 0.2) (layer "B.Cu") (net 3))
 (via blind (at 155.18 111.5675) (size 0.6) (drill 0.3) (layers "F.Cu" "B.Cu") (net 8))
 (segment (start 155.3025 111.5675) (end 155.602031 111.267969) (width 0.2) (layer "B.Cu") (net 8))
 (segment (start 155.18 111.5675) (end 155.3025 111.5675) (width 0.2) (layer "B.Cu") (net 8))
 (segment (start 149.2249 110.2018) (end 150.5906 111.5675) (width 0.2) (layer "B.Cu") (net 8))
 (segment (start 149.2249 109.35) (end 149.2249 110.2018) (width 0.2) (layer "B.Cu") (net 8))
 (segment (start 150.5906 111.5675) (end 155.18 111.5675) (width 0.2) (layer "B.Cu") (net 8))
 (segment (start 155.602031 111.267969) (end 159.537969 111.267969) (width 0.2) (layer "B.Cu") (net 8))
 (segment (start 151.74 100.635) (end 151.725 100.65) (width 0.2) (layer "F.Cu") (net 1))
 (segment (start 155.18 113.3925) (end 151.725 109.9375) (width 0.2) (layer "F.Cu") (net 1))
 (segment (start 149.6825 98.12) (end 152.39 98.12) (width 0.2) (layer "F.Cu") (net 1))
 (segment (start 146.87 113.425) (end 147.65 113.425) (width 0.2) (layer "F.Cu") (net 1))
 (segment (start 142.537969 109.092969) (end 142.537969 107.767969) (width 0.2) (layer "F.Cu") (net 1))
 (segment (start 151.74 98.38) (end 151.74 100.635) (width 0.2) (layer "F.Cu") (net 1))
 (segment (start 152.39 98.12) (end 152.45 98.18) (width 0.2) (layer "F.Cu") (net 1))
 (segment (start 146.87 113.425) (end 142.537969 109.092969) (width 0.2) (layer "F.Cu") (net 1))
 (segment (start 151.94 98.18) (end 151.74 98.38) (width 0.2) (layer "F.Cu") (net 1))
 (segment (start 151.725 109.9375) (end 151.725 109.35) (width 0.2) (layer "F.Cu") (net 1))
 (segment (start 152.45 98.18) (end 151.94 98.18) (width 0.2) (layer "F.Cu") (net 1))
 (segment (start 147.65 113.425) (end 151.725 109.35) (width 0.2) (layer "F.Cu") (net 1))
 (via blind (at 151.725 109.35) (size 0.6) (drill 0.3) (layers "F.Cu" "B.Cu") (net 1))
 (via blind (at 151.725 100.65) (size 0.6) (drill 0.3) (layers "F.Cu" "B.Cu") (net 1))
 (segment (start 142.537969 107.767969) (end 144.7241 105.581838) (width 0.2) (layer "B.Cu") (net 1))
 (segment (start 144.7241 101.7989) (end 147.274 99.249) (width 0.2) (layer "B.Cu") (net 1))
 (segment (start 151.725 99.95) (end 151.725 100.65) (width 0.2) (layer "B.Cu") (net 1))
 (segment (start 144.7241 105.581838) (end 144.7241 101.7989) (width 0.2) (layer "B.Cu") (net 1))
 (segment (start 151.024 99.249) (end 151.725 99.95) (width 0.2) (layer "B.Cu") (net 1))
 (segment (start 147.274 99.249) (end 151.024 99.249) (width 0.2) (layer "B.Cu") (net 1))
 (via blind (at 146.87 111.6) (size 0.6) (drill 0.3) (layers "F.Cu" "B.Cu") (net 2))
 (segment (start 141.336969 107.270498) (end 144.3231 104.284367) (width 0.2) (layer "B.Cu") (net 2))
 (segment (start 153.2749 98.848) (end 158.336969 103.910069) (width 0.2) (layer "B.Cu") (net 2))
 (segment (start 141.336969 108.26544) (end 141.336969 107.270498) (width 0.2) (layer "B.Cu") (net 2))
 (segment (start 144.671529 111.6) (end 141.336969 108.26544) (width 0.2) (layer "B.Cu") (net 2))
 (segment (start 144.3231 101.6328) (end 147.1079 98.848) (width 0.2) (layer "B.Cu") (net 2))
 (segment (start 144.3231 104.284367) (end 144.3231 101.6328) (width 0.2) (layer "B.Cu") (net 2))
 (segment (start 147.975 109.35) (end 147.975 110.495) (width 0.2) (layer "B.Cu") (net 2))
 (segment (start 146.87 111.6) (end 144.671529 111.6) (width 0.2) (layer "B.Cu") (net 2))
 (segment (start 147.975 110.495) (end 146.87 111.6) (width 0.2) (layer "B.Cu") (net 2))
 (segment (start 158.336969 103.910069) (end 158.336969 106.566969) (width 0.2) (layer "B.Cu") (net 2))
 (segment (start 158.336969 106.566969) (end 159.537969 107.767969) (width 0.2) (layer "B.Cu") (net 2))
 (segment (start 147.1079 98.848) (end 153.2749 98.848) (width 0.2) (layer "B.Cu") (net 2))
 (via blind (at 147.8575 98.12) (size 0.6) (drill 0.3) (layers "F.Cu" "B.Cu") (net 5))
 (segment (start 145.185938 98.12) (end 147.8575 98.12) (width 0.2) (layer "B.Cu") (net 5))
 (segment (start 142.537969 100.767969) (end 145.185938 98.12) (width 0.2) (layer "B.Cu") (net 5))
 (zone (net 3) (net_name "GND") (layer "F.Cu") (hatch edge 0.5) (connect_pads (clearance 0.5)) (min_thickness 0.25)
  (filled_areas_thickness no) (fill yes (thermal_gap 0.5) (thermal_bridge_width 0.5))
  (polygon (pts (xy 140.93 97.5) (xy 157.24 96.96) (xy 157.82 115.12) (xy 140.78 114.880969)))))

